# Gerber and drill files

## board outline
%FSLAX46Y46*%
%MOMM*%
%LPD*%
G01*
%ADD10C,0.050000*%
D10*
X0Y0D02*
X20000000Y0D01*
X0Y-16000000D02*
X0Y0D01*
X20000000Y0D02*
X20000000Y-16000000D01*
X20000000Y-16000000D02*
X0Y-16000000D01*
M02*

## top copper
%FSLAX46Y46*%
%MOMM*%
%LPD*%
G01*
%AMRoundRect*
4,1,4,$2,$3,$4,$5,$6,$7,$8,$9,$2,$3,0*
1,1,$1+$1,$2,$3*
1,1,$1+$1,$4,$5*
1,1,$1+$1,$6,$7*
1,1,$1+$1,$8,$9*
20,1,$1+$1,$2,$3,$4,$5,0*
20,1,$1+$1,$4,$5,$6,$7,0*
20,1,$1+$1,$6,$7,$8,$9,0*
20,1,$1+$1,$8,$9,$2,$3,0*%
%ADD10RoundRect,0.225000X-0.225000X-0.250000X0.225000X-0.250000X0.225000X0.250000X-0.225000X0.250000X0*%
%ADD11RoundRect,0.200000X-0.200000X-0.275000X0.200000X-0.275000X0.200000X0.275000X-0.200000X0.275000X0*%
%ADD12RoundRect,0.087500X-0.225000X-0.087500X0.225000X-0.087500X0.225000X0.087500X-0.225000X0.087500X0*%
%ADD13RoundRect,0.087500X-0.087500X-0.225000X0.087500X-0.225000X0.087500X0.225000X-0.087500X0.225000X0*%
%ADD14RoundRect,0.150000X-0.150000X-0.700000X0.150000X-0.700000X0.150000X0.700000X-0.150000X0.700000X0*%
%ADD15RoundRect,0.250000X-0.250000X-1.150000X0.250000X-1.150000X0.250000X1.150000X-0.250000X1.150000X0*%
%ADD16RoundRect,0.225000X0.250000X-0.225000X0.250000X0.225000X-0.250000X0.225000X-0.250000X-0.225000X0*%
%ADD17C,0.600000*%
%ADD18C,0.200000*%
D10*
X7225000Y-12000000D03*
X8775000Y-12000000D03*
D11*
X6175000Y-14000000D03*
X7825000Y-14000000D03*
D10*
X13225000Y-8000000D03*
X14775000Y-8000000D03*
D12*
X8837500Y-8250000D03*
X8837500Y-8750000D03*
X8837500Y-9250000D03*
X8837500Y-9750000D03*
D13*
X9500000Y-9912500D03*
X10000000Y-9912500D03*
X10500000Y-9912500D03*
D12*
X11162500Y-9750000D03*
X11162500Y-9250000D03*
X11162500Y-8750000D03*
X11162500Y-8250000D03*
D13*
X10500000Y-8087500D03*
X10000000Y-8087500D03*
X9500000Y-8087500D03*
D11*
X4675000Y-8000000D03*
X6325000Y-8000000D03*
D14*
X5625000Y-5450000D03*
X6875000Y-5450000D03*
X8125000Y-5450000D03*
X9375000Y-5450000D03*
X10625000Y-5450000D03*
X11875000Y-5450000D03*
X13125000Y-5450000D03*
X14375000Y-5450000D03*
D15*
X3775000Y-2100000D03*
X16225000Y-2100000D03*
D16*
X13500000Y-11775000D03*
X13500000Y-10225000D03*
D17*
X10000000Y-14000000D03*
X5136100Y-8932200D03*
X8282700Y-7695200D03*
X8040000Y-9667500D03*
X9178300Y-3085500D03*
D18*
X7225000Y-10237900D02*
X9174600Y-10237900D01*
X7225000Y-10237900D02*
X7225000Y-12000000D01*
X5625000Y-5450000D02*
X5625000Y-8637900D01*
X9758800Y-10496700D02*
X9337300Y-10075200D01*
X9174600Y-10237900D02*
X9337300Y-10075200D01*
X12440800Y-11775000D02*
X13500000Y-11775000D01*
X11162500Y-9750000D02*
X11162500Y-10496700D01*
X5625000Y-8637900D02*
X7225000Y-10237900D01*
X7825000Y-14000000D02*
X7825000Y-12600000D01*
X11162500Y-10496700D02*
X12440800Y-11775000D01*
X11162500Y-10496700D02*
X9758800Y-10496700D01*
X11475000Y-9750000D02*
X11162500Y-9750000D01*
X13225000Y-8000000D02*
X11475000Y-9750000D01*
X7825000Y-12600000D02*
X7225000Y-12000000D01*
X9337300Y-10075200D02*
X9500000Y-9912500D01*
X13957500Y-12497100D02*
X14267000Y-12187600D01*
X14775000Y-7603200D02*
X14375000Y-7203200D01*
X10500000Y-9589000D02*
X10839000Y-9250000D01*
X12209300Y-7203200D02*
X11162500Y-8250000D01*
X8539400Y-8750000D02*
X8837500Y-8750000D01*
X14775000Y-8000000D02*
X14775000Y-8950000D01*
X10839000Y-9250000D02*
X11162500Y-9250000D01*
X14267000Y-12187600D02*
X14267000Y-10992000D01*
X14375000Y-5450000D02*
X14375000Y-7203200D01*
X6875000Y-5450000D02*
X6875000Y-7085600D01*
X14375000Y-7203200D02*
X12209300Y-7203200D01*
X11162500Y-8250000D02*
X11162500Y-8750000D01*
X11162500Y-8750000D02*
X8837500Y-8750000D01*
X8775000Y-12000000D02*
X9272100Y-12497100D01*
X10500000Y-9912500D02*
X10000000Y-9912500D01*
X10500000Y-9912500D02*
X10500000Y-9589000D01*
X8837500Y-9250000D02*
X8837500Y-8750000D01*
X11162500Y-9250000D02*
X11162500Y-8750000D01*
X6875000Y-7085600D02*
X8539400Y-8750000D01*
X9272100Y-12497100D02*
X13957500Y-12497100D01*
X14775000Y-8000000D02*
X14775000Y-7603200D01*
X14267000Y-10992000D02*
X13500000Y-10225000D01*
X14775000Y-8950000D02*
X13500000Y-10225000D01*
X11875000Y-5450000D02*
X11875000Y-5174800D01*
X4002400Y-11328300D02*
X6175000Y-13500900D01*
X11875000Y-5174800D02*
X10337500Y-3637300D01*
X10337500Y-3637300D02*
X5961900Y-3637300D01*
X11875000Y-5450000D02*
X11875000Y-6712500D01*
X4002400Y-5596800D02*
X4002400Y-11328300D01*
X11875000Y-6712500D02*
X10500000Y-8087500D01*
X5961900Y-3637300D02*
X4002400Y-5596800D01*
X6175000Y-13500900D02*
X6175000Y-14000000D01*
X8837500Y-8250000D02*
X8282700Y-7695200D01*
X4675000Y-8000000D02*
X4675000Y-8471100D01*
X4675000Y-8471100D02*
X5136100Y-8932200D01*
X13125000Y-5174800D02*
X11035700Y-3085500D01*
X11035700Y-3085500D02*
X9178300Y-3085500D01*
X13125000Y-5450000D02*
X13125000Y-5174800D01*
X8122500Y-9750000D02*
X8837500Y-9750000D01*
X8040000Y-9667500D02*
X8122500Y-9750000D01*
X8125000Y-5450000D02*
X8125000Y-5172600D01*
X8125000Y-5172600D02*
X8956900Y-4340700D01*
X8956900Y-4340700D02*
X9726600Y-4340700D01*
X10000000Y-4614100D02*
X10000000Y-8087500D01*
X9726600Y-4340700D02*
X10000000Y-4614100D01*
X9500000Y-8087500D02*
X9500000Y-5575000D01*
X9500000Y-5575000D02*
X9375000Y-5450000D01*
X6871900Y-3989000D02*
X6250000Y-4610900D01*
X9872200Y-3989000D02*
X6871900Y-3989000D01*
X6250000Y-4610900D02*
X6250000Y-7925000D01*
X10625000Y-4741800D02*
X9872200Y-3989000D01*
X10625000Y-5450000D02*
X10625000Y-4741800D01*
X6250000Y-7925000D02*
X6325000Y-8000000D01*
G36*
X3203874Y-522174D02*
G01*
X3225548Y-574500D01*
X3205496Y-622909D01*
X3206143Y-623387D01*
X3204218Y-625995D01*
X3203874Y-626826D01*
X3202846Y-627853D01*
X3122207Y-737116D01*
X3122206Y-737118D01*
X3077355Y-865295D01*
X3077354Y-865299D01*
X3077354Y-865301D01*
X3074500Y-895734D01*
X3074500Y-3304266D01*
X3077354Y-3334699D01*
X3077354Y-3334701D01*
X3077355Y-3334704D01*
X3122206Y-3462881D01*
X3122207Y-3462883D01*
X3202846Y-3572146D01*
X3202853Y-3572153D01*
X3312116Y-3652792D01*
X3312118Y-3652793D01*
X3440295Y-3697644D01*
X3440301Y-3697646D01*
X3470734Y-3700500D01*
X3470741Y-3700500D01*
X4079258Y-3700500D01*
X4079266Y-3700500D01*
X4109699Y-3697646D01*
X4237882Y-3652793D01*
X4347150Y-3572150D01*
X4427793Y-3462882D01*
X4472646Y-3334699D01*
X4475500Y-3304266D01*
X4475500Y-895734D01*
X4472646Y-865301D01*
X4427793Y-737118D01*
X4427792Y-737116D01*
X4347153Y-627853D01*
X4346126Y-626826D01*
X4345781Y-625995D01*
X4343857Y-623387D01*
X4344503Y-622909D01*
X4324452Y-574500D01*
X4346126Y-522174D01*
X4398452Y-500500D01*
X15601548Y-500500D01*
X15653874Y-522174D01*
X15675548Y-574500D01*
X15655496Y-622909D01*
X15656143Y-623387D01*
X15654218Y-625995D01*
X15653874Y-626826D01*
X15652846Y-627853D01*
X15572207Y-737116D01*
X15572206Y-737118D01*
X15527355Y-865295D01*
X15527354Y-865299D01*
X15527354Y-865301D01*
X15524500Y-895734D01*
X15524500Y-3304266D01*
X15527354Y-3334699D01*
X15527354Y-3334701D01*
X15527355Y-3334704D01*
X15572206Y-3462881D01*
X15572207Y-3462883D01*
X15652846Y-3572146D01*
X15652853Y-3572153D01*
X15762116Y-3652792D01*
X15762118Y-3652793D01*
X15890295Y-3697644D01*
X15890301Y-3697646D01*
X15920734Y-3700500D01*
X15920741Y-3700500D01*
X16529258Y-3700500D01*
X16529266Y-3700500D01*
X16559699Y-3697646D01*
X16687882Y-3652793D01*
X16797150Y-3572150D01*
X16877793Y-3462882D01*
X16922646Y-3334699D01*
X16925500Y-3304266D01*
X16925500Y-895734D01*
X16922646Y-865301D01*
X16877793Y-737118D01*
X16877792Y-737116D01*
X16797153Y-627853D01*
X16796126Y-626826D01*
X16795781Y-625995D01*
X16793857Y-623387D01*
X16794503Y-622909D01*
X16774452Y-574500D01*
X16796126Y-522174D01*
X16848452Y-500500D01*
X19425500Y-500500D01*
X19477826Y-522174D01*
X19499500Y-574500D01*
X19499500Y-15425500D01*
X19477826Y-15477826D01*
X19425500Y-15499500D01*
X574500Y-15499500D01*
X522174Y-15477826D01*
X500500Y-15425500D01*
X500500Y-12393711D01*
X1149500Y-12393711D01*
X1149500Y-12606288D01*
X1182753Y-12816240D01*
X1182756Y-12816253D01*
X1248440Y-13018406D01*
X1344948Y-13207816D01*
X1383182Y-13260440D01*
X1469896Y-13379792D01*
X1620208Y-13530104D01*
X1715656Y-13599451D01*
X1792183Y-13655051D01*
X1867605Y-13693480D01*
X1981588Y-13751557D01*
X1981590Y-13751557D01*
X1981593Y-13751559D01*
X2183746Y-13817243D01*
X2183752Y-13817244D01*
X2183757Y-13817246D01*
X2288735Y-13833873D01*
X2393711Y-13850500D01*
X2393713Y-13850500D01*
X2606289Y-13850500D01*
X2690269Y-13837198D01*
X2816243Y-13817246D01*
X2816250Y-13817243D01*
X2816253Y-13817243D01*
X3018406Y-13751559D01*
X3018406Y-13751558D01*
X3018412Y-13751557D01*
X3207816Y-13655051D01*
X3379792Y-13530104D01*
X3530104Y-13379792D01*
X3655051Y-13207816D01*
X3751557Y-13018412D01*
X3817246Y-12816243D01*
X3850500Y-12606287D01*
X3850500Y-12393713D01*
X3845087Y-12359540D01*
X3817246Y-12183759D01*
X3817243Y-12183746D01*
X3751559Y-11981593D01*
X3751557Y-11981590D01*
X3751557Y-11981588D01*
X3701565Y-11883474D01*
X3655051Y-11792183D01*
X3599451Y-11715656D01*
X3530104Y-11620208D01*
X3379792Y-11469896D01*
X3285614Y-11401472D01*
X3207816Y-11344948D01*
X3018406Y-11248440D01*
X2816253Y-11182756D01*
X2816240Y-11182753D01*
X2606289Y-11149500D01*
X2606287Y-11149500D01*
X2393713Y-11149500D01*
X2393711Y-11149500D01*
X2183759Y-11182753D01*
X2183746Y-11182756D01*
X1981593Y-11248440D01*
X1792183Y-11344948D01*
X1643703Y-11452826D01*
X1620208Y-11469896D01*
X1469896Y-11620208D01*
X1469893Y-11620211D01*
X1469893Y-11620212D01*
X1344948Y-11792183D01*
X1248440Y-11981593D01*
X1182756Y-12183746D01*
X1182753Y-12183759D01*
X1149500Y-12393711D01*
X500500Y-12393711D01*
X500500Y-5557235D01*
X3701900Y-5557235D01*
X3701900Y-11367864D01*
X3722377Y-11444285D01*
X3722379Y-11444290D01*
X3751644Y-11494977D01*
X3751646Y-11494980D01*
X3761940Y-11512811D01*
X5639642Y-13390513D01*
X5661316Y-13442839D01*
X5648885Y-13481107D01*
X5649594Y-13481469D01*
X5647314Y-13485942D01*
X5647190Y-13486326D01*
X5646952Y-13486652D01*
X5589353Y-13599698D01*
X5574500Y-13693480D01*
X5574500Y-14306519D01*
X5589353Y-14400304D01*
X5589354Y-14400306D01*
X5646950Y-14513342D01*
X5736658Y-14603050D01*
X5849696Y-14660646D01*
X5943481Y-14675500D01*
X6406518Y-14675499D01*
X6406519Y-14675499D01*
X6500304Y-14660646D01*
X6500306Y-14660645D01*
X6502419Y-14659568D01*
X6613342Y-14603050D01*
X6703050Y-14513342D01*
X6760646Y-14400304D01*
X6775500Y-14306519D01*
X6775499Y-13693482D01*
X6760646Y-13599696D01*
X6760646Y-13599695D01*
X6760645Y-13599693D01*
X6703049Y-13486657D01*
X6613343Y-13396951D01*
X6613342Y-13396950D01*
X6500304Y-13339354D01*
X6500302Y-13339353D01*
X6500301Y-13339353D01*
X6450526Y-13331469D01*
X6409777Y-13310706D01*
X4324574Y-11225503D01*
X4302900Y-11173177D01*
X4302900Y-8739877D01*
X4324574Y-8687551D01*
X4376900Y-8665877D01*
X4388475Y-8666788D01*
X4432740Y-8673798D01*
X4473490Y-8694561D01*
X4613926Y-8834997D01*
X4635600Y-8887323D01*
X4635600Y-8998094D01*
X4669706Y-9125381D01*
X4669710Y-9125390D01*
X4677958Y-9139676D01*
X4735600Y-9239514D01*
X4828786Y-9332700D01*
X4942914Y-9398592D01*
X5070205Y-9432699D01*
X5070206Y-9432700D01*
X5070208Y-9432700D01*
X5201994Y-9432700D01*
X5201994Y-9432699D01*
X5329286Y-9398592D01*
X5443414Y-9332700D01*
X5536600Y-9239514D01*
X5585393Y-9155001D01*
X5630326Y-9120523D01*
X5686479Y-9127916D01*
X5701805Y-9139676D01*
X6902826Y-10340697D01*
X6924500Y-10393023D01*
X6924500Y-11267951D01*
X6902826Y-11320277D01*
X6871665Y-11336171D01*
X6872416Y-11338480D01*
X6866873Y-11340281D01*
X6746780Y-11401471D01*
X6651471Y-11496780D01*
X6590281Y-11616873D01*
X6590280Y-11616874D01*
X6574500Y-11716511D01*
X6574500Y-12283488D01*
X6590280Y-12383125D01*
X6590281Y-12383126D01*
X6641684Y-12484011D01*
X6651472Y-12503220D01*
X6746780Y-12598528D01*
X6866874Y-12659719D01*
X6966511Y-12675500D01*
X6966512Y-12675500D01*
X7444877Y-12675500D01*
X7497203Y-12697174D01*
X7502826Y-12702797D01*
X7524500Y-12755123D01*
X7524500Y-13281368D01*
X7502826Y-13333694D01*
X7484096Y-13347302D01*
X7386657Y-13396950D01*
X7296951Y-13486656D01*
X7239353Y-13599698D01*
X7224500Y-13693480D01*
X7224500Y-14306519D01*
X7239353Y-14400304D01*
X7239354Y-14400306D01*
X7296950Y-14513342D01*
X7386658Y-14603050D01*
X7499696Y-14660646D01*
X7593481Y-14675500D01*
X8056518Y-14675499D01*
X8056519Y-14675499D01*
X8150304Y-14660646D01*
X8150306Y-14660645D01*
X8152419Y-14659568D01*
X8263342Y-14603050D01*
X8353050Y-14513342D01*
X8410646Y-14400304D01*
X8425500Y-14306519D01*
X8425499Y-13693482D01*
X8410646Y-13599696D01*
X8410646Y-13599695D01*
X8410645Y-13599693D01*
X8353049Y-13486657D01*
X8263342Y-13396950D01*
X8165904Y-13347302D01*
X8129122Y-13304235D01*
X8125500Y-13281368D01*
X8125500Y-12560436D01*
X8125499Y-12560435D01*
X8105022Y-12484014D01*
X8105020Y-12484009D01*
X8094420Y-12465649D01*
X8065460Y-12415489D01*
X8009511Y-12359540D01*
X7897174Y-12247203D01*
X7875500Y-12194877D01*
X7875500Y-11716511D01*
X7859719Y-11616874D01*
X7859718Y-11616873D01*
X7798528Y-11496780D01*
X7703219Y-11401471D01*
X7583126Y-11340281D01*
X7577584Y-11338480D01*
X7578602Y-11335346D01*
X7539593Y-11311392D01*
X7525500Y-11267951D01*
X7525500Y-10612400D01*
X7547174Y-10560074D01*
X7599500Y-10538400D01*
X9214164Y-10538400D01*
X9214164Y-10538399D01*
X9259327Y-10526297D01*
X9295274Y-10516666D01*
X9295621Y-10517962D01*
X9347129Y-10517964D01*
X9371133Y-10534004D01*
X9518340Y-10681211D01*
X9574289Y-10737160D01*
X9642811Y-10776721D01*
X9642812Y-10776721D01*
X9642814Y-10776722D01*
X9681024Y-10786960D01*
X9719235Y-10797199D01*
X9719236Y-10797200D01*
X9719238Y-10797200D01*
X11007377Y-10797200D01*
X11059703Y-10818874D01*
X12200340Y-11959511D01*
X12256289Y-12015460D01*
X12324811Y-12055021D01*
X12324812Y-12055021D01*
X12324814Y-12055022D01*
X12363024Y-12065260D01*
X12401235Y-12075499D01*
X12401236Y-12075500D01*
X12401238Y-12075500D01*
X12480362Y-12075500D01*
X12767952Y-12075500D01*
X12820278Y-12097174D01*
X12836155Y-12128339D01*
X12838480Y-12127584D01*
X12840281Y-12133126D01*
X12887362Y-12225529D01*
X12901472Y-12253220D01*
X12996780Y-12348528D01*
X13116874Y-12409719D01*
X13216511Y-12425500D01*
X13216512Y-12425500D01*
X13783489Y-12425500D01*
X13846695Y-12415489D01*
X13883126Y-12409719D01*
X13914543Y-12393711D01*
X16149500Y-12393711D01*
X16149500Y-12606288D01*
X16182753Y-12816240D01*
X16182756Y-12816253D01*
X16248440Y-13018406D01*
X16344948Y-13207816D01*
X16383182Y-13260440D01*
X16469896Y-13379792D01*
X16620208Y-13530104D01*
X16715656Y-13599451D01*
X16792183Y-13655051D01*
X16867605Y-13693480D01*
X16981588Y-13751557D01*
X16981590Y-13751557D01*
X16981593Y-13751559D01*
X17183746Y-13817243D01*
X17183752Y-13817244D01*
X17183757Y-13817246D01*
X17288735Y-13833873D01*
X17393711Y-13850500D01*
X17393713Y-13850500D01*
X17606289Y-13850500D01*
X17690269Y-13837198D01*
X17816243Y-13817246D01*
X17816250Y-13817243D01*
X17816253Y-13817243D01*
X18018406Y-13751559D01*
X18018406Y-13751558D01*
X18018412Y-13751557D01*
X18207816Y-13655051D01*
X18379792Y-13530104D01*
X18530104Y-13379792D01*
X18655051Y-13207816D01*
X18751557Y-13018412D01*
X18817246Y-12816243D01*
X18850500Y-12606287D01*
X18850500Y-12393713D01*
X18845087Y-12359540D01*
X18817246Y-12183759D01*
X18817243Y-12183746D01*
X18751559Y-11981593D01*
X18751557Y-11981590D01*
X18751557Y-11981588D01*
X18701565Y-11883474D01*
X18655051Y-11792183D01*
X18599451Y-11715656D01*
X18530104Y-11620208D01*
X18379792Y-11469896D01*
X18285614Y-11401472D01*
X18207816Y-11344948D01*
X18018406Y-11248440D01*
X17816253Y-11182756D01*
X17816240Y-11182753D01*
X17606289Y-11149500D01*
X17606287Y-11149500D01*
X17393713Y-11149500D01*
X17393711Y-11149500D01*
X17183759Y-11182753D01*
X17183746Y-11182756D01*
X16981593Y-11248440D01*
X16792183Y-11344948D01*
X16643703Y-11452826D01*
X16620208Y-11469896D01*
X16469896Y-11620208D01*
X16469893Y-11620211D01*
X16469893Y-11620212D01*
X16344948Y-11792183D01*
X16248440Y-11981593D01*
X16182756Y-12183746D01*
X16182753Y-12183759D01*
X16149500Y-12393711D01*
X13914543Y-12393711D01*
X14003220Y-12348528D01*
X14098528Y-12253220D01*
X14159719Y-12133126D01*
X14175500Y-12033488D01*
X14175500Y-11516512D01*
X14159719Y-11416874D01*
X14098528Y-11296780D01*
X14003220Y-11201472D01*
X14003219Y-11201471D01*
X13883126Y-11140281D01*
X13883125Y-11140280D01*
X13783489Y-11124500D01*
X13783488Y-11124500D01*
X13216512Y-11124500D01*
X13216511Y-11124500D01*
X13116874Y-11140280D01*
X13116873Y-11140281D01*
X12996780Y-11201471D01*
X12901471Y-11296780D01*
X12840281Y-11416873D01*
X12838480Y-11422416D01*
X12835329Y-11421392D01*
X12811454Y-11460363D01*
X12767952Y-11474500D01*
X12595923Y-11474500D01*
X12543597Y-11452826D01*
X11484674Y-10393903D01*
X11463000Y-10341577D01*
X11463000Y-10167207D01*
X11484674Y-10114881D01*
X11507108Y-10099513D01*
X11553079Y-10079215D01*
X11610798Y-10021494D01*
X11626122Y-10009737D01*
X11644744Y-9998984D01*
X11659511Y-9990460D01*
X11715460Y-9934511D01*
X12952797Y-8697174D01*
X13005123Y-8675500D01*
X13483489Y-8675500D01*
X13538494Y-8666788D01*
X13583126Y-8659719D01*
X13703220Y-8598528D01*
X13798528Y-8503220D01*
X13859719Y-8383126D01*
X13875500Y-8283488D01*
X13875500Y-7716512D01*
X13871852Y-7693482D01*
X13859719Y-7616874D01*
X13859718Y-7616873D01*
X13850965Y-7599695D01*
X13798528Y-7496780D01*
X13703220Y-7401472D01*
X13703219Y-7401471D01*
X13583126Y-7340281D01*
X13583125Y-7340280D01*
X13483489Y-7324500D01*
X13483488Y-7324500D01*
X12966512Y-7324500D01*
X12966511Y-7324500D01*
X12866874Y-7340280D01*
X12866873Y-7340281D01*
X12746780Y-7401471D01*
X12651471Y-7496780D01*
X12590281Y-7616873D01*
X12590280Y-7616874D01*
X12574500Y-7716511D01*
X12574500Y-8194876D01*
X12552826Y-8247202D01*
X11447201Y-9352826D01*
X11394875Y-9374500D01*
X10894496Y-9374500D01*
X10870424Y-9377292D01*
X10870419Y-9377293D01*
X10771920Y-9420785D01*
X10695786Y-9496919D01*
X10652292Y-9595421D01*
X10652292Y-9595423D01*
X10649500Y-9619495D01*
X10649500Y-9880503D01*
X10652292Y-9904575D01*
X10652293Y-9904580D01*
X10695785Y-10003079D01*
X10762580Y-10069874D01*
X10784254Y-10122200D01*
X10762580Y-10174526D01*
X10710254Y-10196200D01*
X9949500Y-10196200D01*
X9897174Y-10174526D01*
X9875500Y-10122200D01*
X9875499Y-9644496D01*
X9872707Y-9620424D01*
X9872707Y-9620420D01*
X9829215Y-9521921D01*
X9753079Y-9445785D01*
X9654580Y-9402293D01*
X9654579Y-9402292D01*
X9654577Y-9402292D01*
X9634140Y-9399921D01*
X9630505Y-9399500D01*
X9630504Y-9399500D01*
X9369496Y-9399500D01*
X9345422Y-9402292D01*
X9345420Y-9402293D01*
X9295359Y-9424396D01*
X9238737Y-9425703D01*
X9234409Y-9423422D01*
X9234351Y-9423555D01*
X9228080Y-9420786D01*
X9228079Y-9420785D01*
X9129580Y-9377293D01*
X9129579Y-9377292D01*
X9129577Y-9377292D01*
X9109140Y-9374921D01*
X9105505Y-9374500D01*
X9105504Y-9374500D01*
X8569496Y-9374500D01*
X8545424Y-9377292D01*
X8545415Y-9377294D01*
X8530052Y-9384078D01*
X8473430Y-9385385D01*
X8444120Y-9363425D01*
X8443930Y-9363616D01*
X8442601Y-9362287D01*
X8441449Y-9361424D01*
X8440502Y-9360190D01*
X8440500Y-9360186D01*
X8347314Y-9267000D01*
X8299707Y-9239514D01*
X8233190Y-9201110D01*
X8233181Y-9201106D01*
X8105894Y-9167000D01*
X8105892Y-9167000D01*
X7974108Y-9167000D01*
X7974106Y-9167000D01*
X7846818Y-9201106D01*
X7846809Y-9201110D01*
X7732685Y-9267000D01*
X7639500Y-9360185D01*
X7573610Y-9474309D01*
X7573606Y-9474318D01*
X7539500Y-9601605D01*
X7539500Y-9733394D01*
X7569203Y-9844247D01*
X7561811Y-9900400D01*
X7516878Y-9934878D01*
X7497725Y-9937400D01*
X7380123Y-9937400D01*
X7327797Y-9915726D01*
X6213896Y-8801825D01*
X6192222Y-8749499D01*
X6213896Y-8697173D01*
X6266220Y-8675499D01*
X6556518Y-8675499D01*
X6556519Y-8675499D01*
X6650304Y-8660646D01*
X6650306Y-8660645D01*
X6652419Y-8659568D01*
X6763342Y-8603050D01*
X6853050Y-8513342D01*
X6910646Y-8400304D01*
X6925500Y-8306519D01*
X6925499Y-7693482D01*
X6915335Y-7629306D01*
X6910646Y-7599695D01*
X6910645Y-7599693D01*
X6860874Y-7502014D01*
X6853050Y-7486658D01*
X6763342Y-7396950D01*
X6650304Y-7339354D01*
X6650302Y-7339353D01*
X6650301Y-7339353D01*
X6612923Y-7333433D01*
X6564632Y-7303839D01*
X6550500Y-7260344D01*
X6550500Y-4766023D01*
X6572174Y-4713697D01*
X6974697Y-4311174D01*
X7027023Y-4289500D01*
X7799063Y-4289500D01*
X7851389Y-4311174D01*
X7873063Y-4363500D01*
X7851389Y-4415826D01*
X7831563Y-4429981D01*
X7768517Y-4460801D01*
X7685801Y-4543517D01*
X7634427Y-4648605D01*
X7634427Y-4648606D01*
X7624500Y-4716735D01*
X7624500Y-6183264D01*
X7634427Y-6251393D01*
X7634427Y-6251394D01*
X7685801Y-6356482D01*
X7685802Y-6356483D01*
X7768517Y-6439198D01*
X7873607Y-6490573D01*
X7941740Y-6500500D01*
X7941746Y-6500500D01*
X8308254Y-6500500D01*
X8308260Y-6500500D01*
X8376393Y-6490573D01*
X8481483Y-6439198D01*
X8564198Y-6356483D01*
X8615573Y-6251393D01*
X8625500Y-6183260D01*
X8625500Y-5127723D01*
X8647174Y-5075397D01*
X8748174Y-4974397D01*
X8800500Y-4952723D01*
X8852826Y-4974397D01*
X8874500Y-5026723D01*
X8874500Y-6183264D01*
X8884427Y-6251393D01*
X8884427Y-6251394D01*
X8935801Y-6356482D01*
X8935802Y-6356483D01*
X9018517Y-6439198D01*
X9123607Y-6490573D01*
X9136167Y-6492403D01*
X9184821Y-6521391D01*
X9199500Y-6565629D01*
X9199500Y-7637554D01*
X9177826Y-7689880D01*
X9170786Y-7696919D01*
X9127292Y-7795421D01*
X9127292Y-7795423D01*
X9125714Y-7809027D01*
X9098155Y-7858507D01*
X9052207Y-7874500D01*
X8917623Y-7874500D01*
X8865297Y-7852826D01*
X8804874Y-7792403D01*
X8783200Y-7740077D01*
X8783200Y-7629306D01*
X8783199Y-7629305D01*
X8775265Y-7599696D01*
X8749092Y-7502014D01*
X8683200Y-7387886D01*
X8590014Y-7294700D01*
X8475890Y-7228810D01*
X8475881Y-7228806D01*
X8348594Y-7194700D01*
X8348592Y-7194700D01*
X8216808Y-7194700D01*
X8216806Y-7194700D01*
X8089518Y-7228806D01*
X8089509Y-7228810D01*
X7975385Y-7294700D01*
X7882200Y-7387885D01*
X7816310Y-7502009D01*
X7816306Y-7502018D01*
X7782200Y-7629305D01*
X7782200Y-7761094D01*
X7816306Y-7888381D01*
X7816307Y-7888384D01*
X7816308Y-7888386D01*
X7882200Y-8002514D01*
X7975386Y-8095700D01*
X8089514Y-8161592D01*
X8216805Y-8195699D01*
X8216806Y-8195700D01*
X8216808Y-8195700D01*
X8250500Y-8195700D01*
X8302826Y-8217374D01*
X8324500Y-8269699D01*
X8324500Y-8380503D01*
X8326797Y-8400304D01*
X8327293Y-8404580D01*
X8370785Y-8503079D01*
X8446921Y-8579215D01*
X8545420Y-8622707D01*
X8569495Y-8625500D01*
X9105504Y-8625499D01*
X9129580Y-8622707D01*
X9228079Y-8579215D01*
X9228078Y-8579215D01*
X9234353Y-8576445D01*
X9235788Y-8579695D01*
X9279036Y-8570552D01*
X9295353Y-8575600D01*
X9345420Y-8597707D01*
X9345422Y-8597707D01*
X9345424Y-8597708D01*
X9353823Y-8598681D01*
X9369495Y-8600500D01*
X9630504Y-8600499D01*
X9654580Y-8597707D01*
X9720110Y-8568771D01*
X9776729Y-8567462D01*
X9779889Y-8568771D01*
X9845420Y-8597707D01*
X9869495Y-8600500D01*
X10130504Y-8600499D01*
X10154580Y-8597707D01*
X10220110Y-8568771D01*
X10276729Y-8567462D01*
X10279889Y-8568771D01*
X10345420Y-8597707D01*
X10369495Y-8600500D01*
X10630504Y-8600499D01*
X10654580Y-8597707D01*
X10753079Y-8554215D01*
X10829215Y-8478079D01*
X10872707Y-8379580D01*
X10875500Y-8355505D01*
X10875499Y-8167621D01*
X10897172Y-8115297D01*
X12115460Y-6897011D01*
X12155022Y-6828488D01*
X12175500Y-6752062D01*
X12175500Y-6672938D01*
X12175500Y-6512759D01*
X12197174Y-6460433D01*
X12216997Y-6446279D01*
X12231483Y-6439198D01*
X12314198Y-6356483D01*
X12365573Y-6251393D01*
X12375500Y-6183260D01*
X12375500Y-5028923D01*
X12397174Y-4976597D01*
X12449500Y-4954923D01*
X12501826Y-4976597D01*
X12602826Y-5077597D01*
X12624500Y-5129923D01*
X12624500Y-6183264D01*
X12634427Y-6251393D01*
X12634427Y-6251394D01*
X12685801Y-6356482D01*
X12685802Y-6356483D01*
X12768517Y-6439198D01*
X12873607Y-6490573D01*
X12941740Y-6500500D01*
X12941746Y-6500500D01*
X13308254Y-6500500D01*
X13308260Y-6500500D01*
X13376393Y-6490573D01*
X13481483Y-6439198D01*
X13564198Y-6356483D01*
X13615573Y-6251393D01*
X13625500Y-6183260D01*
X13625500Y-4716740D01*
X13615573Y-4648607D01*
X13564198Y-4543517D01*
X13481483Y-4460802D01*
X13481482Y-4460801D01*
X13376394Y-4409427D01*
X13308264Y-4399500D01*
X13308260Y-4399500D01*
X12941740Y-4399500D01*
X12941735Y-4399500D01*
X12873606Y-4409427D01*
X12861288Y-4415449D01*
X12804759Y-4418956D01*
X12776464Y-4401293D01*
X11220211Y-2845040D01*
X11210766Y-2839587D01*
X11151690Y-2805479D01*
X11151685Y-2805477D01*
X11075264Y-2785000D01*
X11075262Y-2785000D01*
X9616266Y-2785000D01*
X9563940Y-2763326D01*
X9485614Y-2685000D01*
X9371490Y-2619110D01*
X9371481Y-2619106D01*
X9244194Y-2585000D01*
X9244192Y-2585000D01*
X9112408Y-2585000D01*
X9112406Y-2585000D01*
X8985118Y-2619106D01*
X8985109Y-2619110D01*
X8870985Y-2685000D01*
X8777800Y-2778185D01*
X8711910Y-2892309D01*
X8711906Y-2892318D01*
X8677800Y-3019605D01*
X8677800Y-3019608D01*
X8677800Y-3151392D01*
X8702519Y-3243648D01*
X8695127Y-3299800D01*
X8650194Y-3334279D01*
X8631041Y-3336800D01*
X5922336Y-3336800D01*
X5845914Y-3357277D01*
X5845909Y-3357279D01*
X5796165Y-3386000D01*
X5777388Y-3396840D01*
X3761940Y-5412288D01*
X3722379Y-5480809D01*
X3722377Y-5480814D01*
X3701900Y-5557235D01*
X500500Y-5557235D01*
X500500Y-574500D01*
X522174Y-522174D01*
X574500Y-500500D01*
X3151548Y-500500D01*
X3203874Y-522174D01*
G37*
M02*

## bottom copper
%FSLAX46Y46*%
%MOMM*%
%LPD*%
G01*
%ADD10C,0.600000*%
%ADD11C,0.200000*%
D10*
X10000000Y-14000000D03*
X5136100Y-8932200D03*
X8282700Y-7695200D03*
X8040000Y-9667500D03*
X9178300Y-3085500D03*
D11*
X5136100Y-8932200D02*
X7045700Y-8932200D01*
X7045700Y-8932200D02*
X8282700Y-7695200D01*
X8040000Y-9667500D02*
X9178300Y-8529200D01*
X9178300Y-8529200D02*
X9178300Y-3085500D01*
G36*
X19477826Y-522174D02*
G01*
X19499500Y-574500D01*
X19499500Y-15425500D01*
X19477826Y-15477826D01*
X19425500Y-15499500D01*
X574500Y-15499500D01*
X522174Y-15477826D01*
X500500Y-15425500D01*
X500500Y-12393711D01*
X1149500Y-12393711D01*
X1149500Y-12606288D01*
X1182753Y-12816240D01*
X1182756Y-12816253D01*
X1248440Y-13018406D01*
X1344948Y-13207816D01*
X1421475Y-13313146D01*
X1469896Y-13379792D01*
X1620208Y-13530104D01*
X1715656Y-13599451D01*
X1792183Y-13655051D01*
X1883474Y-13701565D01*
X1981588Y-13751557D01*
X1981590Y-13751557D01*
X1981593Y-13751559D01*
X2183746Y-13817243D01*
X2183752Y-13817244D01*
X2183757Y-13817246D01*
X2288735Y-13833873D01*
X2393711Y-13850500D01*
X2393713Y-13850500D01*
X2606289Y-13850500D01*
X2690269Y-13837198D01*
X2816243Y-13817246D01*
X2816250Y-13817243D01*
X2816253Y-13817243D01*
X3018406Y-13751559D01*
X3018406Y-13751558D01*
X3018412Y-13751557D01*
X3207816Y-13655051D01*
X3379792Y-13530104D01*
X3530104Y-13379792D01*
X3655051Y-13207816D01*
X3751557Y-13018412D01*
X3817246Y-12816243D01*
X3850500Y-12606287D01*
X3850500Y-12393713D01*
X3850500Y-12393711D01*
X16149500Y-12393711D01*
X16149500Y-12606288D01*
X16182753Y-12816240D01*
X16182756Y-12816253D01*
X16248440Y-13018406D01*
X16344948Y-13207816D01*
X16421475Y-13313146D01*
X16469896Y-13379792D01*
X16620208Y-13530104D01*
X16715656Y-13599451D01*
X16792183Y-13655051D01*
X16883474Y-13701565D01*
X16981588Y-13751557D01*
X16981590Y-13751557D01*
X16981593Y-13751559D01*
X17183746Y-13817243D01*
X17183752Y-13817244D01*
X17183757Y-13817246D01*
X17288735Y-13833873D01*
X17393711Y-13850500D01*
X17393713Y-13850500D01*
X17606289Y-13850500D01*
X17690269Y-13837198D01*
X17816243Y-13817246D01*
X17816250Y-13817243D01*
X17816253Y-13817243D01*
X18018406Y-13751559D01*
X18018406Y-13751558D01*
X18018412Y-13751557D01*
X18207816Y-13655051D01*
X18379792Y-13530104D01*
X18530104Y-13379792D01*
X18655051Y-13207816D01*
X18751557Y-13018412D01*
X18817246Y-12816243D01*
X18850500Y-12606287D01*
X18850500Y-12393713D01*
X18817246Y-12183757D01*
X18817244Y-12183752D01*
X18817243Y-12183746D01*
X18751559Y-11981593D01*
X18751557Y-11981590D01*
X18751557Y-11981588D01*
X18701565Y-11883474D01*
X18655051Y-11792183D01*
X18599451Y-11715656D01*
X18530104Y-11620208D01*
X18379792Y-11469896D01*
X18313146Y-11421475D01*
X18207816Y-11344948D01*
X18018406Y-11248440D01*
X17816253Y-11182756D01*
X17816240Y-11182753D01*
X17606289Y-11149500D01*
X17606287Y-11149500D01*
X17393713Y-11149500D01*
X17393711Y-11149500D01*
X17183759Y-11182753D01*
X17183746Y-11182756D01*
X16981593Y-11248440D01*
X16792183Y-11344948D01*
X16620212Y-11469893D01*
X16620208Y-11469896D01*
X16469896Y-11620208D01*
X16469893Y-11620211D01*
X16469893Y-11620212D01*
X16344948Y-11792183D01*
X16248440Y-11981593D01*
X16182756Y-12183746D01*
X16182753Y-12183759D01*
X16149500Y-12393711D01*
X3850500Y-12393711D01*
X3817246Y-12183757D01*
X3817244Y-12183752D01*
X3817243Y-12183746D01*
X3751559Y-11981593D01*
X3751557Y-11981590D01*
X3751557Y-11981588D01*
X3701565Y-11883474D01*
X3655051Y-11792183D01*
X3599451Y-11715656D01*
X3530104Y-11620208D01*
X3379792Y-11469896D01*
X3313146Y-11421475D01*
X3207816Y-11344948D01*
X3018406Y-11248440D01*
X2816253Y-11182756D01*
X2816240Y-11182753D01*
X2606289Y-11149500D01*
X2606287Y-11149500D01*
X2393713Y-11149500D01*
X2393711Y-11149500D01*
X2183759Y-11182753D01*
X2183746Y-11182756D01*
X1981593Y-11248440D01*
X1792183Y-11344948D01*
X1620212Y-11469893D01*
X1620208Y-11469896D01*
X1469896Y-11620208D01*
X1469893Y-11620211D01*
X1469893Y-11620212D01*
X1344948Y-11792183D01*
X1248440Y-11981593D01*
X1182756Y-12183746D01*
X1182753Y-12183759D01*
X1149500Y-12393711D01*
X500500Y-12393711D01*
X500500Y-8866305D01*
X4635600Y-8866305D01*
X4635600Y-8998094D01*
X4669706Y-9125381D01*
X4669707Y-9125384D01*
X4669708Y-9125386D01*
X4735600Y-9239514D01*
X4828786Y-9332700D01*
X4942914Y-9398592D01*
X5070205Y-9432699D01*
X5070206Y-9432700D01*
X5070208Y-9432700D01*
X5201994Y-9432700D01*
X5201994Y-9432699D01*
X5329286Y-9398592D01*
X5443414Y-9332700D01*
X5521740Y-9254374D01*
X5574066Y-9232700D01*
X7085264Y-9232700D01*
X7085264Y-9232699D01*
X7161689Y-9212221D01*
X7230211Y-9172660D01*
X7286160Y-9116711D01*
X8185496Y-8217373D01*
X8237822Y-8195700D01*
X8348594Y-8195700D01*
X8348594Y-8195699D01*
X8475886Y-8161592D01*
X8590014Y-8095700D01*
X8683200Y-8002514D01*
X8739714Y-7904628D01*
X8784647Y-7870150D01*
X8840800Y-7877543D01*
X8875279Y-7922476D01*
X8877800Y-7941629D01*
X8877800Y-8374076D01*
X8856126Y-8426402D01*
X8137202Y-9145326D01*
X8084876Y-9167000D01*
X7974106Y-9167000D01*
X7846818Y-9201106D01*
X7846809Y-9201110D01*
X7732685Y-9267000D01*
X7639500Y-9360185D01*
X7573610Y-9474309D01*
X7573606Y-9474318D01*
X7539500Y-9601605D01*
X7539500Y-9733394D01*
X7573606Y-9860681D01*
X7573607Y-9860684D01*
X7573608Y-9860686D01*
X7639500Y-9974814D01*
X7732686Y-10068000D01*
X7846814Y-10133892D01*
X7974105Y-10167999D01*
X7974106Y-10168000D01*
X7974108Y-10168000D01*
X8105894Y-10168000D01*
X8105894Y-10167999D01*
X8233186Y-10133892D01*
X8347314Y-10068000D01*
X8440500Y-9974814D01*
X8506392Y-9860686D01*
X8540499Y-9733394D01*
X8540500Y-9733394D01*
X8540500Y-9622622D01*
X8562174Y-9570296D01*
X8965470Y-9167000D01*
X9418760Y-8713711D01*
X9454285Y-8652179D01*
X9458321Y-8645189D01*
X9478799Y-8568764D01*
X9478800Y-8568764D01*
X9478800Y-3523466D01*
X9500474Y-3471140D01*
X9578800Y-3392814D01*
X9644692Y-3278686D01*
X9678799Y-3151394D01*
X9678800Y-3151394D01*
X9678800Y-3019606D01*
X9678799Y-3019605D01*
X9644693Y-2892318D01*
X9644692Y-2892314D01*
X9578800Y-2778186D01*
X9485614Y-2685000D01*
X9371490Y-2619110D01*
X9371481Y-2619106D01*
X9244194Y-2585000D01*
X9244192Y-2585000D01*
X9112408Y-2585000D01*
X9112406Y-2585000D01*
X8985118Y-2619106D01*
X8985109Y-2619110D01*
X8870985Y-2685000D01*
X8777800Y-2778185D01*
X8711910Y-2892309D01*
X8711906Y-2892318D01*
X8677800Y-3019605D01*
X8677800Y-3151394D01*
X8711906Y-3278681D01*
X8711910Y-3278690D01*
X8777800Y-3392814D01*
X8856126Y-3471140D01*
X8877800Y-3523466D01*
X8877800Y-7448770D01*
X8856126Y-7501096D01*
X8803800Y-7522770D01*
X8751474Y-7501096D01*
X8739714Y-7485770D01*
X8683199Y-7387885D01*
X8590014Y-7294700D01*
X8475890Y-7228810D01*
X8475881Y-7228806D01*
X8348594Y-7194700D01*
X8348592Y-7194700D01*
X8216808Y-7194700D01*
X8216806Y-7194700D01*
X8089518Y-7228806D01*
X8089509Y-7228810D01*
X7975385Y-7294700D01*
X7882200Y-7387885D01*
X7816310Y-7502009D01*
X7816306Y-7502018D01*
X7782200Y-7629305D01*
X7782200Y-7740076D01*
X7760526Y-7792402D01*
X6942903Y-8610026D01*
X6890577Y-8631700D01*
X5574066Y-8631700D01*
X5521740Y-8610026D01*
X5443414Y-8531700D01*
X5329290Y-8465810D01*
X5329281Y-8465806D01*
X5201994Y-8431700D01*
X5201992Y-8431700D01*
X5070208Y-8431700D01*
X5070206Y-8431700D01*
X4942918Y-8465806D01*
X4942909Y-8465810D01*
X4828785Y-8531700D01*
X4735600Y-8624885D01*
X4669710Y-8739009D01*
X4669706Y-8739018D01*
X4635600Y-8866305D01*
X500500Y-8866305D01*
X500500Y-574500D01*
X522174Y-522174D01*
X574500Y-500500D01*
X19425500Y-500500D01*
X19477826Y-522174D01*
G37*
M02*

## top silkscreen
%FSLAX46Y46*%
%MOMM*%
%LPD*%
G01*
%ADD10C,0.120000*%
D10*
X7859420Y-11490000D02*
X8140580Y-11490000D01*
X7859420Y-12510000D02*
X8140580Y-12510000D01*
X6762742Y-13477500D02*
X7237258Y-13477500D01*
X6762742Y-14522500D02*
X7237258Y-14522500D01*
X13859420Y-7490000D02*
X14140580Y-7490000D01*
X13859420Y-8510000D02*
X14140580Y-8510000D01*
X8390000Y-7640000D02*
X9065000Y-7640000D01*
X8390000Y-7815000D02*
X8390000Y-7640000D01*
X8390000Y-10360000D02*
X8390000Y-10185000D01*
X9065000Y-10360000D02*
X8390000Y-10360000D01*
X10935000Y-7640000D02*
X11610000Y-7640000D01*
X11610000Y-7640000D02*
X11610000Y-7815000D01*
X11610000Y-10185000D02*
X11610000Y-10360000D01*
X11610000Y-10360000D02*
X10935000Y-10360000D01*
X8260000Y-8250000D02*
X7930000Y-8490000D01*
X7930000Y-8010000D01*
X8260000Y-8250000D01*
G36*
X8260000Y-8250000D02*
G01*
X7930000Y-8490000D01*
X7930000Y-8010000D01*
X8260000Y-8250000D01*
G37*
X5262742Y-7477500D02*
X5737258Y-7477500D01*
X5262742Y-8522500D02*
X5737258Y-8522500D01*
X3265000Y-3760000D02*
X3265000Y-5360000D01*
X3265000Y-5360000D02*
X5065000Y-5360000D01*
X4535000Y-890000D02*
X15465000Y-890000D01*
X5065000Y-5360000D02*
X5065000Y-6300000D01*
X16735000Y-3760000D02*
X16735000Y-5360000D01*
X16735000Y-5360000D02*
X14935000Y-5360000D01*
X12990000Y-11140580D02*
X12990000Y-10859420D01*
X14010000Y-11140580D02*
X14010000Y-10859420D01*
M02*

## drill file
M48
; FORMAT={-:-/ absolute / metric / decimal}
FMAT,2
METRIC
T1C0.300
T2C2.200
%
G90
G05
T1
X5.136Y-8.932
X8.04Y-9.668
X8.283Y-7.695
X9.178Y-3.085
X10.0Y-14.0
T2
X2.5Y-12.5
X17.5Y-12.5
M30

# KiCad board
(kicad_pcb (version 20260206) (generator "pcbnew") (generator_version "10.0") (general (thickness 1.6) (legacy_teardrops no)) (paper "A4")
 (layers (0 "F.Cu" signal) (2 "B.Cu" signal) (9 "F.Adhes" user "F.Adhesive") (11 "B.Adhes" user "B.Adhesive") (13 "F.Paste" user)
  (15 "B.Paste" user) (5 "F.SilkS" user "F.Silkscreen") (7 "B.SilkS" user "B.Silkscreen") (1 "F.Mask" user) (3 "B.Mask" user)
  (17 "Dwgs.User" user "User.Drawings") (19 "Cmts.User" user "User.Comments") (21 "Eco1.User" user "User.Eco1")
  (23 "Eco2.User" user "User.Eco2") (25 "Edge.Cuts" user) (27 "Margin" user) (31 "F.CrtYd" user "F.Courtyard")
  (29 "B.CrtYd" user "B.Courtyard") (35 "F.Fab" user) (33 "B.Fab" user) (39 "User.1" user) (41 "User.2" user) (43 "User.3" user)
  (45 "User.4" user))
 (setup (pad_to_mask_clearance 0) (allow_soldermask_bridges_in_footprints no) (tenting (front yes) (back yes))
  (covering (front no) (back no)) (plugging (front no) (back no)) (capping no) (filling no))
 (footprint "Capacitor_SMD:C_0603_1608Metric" (layer "F.Cu") (at 8 12)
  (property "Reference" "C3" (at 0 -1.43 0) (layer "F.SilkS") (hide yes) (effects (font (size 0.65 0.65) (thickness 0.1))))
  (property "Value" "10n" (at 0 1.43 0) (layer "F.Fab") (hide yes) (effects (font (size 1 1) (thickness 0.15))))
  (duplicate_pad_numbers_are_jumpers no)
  (fp_line (start -0.14058 -0.51) (end 0.14058 -0.51) (stroke (width 0.12) (type solid)) (layer "F.SilkS"))
  (fp_line (start -0.14058 0.51) (end 0.14058 0.51) (stroke (width 0.12) (type solid)) (layer "F.SilkS"))
  (pad "1" smd roundrect (at -0.775 0) (size 0.9 0.95) (layers "F.Cu" "F.Mask" "F.Paste") (roundrect_rratio 0.25) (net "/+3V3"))
  (pad "2" smd roundrect (at 0.775 0) (size 0.9 0.95) (layers "F.Cu" "F.Mask" "F.Paste") (roundrect_rratio 0.25) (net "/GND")
   (zone_connect 2)))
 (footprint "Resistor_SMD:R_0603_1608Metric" (layer "F.Cu") (at 7 14)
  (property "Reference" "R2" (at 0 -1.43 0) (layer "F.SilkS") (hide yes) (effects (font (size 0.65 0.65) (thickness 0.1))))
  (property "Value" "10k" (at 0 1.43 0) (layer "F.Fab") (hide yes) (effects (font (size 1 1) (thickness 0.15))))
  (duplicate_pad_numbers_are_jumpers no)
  (fp_line (start -0.237258 -0.5225) (end 0.237258 -0.5225) (stroke (width 0.12) (type solid)) (layer "F.SilkS"))
  (fp_line (start -0.237258 0.5225) (end 0.237258 0.5225) (stroke (width 0.12) (type solid)) (layer "F.SilkS"))
  (pad "1" smd roundrect (at -0.825 0) (size 0.8 0.95) (layers "F.Cu" "F.Mask" "F.Paste") (roundrect_rratio 0.25) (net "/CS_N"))
  (pad "2" smd roundrect (at 0.825 0) (size 0.8 0.95) (layers "F.Cu" "F.Mask" "F.Paste") (roundrect_rratio 0.25) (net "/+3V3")))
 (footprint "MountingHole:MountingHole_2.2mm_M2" (layer "F.Cu") (at 2.5 12.5)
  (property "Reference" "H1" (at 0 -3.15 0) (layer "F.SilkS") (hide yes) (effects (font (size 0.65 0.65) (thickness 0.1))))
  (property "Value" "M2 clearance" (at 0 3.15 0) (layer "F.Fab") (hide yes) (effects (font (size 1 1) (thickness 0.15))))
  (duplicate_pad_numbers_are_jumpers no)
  (pad "" np_thru_hole circle (at 0 0) (size 2.2 2.2) (drill 2.2) (layers "*.Cu" "*.Mask")))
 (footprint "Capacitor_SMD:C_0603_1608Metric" (layer "F.Cu") (at 14 8)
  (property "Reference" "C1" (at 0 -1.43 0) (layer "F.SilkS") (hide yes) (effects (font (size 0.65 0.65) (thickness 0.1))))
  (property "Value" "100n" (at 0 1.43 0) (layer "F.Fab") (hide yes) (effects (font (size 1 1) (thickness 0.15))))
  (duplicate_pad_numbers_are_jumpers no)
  (fp_line (start -0.14058 -0.51) (end 0.14058 -0.51) (stroke (width 0.12) (type solid)) (layer "F.SilkS"))
  (fp_line (start -0.14058 0.51) (end 0.14058 0.51) (stroke (width 0.12) (type solid)) (layer "F.SilkS"))
  (pad "1" smd roundrect (at -0.775 0) (size 0.9 0.95) (layers "F.Cu" "F.Mask" "F.Paste") (roundrect_rratio 0.25) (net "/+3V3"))
  (pad "2" smd roundrect (at 0.775 0) (size 0.9 0.95) (layers "F.Cu" "F.Mask" "F.Paste") (roundrect_rratio 0.25) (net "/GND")
   (zone_connect 2)))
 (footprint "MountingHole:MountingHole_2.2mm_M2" (layer "F.Cu") (at 17.5 12.5)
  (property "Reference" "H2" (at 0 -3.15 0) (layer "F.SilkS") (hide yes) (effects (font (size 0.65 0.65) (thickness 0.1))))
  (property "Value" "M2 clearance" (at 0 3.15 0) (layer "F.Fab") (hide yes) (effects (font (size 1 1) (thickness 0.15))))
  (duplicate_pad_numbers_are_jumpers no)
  (pad "" np_thru_hole circle (at 0 0) (size 2.2 2.2) (drill 2.2) (layers "*.Cu" "*.Mask")))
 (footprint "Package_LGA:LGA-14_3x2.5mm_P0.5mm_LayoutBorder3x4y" (layer "F.Cu") (at 10 9)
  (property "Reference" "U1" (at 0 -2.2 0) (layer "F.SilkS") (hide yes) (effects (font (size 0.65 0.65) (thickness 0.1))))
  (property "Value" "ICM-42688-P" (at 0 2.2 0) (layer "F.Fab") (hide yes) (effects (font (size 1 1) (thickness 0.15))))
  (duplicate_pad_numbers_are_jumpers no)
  (fp_line (start -1.61 -1.36) (end -0.935 -1.36) (stroke (width 0.12) (type solid)) (layer "F.SilkS"))
  (fp_line (start -1.61 -1.185) (end -1.61 -1.36) (stroke (width 0.12) (type solid)) (layer "F.SilkS"))
  (fp_line (start -1.61 1.36) (end -1.61 1.185) (stroke (width 0.12) (type solid)) (layer "F.SilkS"))
  (fp_line (start -0.935 1.36) (end -1.61 1.36) (stroke (width 0.12) (type solid)) (layer "F.SilkS"))
  (fp_line (start 0.935 -1.36) (end 1.61 -1.36) (stroke (width 0.12) (type solid)) (layer "F.SilkS"))
  (fp_line (start 1.61 -1.36) (end 1.61 -1.185) (stroke (width 0.12) (type solid)) (layer "F.SilkS"))
  (fp_line (start 1.61 1.185) (end 1.61 1.36) (stroke (width 0.12) (type solid)) (layer "F.SilkS"))
  (fp_line (start 1.61 1.36) (end 0.935 1.36) (stroke (width 0.12) (type solid)) (layer "F.SilkS"))
  (fp_poly (pts (xy -1.74 -0.75) (xy -2.07 -0.51) (xy -2.07 -0.99)) (stroke (width 0.12) (type solid)) (fill yes) (layer "F.SilkS"))
  (pad "1" smd roundrect (at -1.1625 -0.75) (size 0.625 0.35) (layers "F.Cu" "F.Mask" "F.Paste") (roundrect_rratio 0.25) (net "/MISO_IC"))
  (pad "2" smd roundrect (at -1.1625 -0.25) (size 0.625 0.35) (layers "F.Cu" "F.Mask" "F.Paste") (roundrect_rratio 0.25) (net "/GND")
   (zone_connect 2))
  (pad "3" smd roundrect (at -1.1625 0.25) (size 0.625 0.35) (layers "F.Cu" "F.Mask" "F.Paste") (roundrect_rratio 0.25) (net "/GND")
   (zone_connect 2))
  (pad "4" smd roundrect (at -1.1625 0.75) (size 0.625 0.35) (layers "F.Cu" "F.Mask" "F.Paste") (roundrect_rratio 0.25) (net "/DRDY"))
  (pad "5" smd roundrect (at -0.5 0.9125) (size 0.35 0.625) (layers "F.Cu" "F.Mask" "F.Paste") (roundrect_rratio 0.25) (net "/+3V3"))
  (pad "6" smd roundrect (at 0 0.9125) (size 0.35 0.625) (layers "F.Cu" "F.Mask" "F.Paste") (roundrect_rratio 0.25) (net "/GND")
   (zone_connect 2))
  (pad "7" smd roundrect (at 0.5 0.9125) (size 0.35 0.625) (layers "F.Cu" "F.Mask" "F.Paste") (roundrect_rratio 0.25) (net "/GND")
   (zone_connect 2))
  (pad "8" smd roundrect (at 1.1625 0.75) (size 0.625 0.35) (layers "F.Cu" "F.Mask" "F.Paste") (roundrect_rratio 0.25) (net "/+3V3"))
  (pad "9" smd roundrect (at 1.1625 0.25) (size 0.625 0.35) (layers "F.Cu" "F.Mask" "F.Paste") (roundrect_rratio 0.25) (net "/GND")
   (zone_connect 2))
  (pad "10" smd roundrect (at 1.1625 -0.25) (size 0.625 0.35) (layers "F.Cu" "F.Mask" "F.Paste") (roundrect_rratio 0.25) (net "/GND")
   (zone_connect 2))
  (pad "11" smd roundrect (at 1.1625 -0.75) (size 0.625 0.35) (layers "F.Cu" "F.Mask" "F.Paste") (roundrect_rratio 0.25) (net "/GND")
   (zone_connect 2))
  (pad "12" smd roundrect (at 0.5 -0.9125) (size 0.35 0.625) (layers "F.Cu" "F.Mask" "F.Paste") (roundrect_rratio 0.25) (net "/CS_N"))
  (pad "13" smd roundrect (at 0 -0.9125) (size 0.35 0.625) (layers "F.Cu" "F.Mask" "F.Paste") (roundrect_rratio 0.25) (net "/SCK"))
  (pad "14" smd roundrect (at -0.5 -0.9125) (size 0.35 0.625) (layers "F.Cu" "F.Mask" "F.Paste") (roundrect_rratio 0.25) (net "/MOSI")))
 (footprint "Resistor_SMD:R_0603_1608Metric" (layer "F.Cu") (at 5.5 8)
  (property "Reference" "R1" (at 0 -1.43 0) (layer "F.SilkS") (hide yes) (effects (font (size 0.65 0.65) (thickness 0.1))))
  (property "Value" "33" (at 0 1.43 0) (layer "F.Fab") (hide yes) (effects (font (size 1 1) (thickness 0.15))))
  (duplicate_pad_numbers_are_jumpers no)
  (fp_line (start -0.237258 -0.5225) (end 0.237258 -0.5225) (stroke (width 0.12) (type solid)) (layer "F.SilkS"))
  (fp_line (start -0.237258 0.5225) (end 0.237258 0.5225) (stroke (width 0.12) (type solid)) (layer "F.SilkS"))
  (pad "1" smd roundrect (at -0.825 0) (size 0.8 0.95) (layers "F.Cu" "F.Mask" "F.Paste") (roundrect_rratio 0.25) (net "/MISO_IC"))
  (pad "2" smd roundrect (at 0.825 0) (size 0.8 0.95) (layers "F.Cu" "F.Mask" "F.Paste") (roundrect_rratio 0.25) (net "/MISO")))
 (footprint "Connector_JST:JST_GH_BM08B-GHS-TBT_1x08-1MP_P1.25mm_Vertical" (layer "F.Cu") (at 10 3.5)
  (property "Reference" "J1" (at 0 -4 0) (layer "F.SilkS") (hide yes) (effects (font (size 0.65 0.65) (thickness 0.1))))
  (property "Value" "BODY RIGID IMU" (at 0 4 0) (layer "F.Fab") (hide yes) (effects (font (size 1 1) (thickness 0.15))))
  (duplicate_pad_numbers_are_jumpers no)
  (fp_line (start -6.735 0.26) (end -6.735 1.86) (stroke (width 0.12) (type solid)) (layer "F.SilkS"))
  (fp_line (start -6.735 1.86) (end -4.935 1.86) (stroke (width 0.12) (type solid)) (layer "F.SilkS"))
  (fp_line (start -5.465 -2.61) (end 5.465 -2.61) (stroke (width 0.12) (type solid)) (layer "F.SilkS"))
  (fp_line (start -4.935 1.86) (end -4.935 2.8) (stroke (width 0.12) (type solid)) (layer "F.SilkS"))
  (fp_line (start 6.735 0.26) (end 6.735 1.86) (stroke (width 0.12) (type solid)) (layer "F.SilkS"))
  (fp_line (start 6.735 1.86) (end 4.935 1.86) (stroke (width 0.12) (type solid)) (layer "F.SilkS"))
  (pad "1" smd roundrect (at -4.375 1.95) (size 0.6 1.7) (layers "F.Cu" "F.Mask" "F.Paste") (roundrect_rratio 0.25) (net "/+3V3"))
  (pad "2" smd roundrect (at -3.125 1.95) (size 0.6 1.7) (layers "F.Cu" "F.Mask" "F.Paste") (roundrect_rratio 0.25) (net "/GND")
   (zone_connect 2))
  (pad "3" smd roundrect (at -1.875 1.95) (size 0.6 1.7) (layers "F.Cu" "F.Mask" "F.Paste") (roundrect_rratio 0.25) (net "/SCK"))
  (pad "4" smd roundrect (at -0.625 1.95) (size 0.6 1.7) (layers "F.Cu" "F.Mask" "F.Paste") (roundrect_rratio 0.25) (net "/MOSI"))
  (pad "5" smd roundrect (at 0.625 1.95) (size 0.6 1.7) (layers "F.Cu" "F.Mask" "F.Paste") (roundrect_rratio 0.25) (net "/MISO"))
  (pad "6" smd roundrect (at 1.875 1.95) (size 0.6 1.7) (layers "F.Cu" "F.Mask" "F.Paste") (roundrect_rratio 0.25) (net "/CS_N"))
  (pad "7" smd roundrect (at 3.125 1.95) (size 0.6 1.7) (layers "F.Cu" "F.Mask" "F.Paste") (roundrect_rratio 0.25) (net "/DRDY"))
  (pad "8" smd roundrect (at 4.375 1.95) (size 0.6 1.7) (layers "F.Cu" "F.Mask" "F.Paste") (roundrect_rratio 0.25) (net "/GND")
   (zone_connect 2))
  (pad "MP" smd roundrect (at -6.225 -1.4) (size 1 2.8) (layers "F.Cu" "F.Mask" "F.Paste") (roundrect_rratio 0.25))
  (pad "MP" smd roundrect (at 6.225 -1.4) (size 1 2.8) (layers "F.Cu" "F.Mask" "F.Paste") (roundrect_rratio 0.25)))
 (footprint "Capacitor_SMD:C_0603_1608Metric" (layer "F.Cu") (at 13.5 11 90)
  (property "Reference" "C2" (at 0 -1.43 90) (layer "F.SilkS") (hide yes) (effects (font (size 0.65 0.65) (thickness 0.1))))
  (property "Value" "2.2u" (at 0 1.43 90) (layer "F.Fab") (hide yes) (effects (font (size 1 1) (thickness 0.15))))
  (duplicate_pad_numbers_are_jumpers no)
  (fp_line (start -0.14058 -0.51) (end 0.14058 -0.51) (stroke (width 0.12) (type solid)) (layer "F.SilkS"))
  (fp_line (start -0.14058 0.51) (end 0.14058 0.51) (stroke (width 0.12) (type solid)) (layer "F.SilkS"))
  (pad "1" smd roundrect (at -0.775 0 90) (size 0.9 0.95) (layers "F.Cu" "F.Mask" "F.Paste") (roundrect_rratio 0.25) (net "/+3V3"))
  (pad "2" smd roundrect (at 0.775 0 90) (size 0.9 0.95) (layers "F.Cu" "F.Mask" "F.Paste") (roundrect_rratio 0.25) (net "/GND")
   (zone_connect 2)))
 (gr_line (start 0 0) (end 20 0) (stroke (width 0.05) (type default)) (layer "Edge.Cuts"))
 (gr_line (start 0 16) (end 0 0) (stroke (width 0.05) (type default)) (layer "Edge.Cuts"))
 (gr_line (start 20 0) (end 20 16) (stroke (width 0.05) (type default)) (layer "Edge.Cuts"))
 (gr_line (start 20 16) (end 0 16) (stroke (width 0.05) (type default)) (layer "Edge.Cuts"))
 (segment (start 7.225 10.2379) (end 9.1746 10.2379) (width 0.2) (layer "F.Cu") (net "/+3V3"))
 (segment (start 7.225 10.2379) (end 7.225 12) (width 0.2) (layer "F.Cu") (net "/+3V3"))
 (segment (start 5.625 5.45) (end 5.625 8.6379) (width 0.2) (layer "F.Cu") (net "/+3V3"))
 (segment (start 9.7588 10.4967) (end 9.3373 10.0752) (width 0.2) (layer "F.Cu") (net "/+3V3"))
 (segment (start 9.1746 10.2379) (end 9.3373 10.0752) (width 0.2) (layer "F.Cu") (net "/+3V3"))
 (segment (start 12.4408 11.775) (end 13.5 11.775) (width 0.2) (layer "F.Cu") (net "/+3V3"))
 (segment (start 11.1625 9.75) (end 11.1625 10.4967) (width 0.2) (layer "F.Cu") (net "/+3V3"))
 (segment (start 5.625 8.6379) (end 7.225 10.2379) (width 0.2) (layer "F.Cu") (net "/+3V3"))
 (segment (start 7.825 14) (end 7.825 12.6) (width 0.2) (layer "F.Cu") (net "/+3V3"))
 (segment (start 11.1625 10.4967) (end 12.4408 11.775) (width 0.2) (layer "F.Cu") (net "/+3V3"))
 (segment (start 11.1625 10.4967) (end 9.7588 10.4967) (width 0.2) (layer "F.Cu") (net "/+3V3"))
 (segment (start 11.475 9.75) (end 11.1625 9.75) (width 0.2) (layer "F.Cu") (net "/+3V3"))
 (segment (start 13.225 8) (end 11.475 9.75) (width 0.2) (layer "F.Cu") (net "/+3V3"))
 (segment (start 7.825 12.6) (end 7.225 12) (width 0.2) (layer "F.Cu") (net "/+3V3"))
 (segment (start 9.3373 10.0752) (end 9.5 9.9125) (width 0.2) (layer "F.Cu") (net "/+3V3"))
 (segment (start 13.9575 12.4971) (end 14.267 12.1876) (width 0.2) (layer "F.Cu") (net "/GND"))
 (segment (start 14.775 7.6032) (end 14.375 7.2032) (width 0.2) (layer "F.Cu") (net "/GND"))
 (segment (start 10.5 9.589) (end 10.839 9.25) (width 0.2) (layer "F.Cu") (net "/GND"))
 (segment (start 12.2093 7.2032) (end 11.1625 8.25) (width 0.2) (layer "F.Cu") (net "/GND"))
 (segment (start 8.5394 8.75) (end 8.8375 8.75) (width 0.2) (layer "F.Cu") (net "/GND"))
 (segment (start 14.775 8) (end 14.775 8.95) (width 0.2) (layer "F.Cu") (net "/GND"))
 (segment (start 10.839 9.25) (end 11.1625 9.25) (width 0.2) (layer "F.Cu") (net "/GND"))
 (segment (start 14.267 12.1876) (end 14.267 10.992) (width 0.2) (layer "F.Cu") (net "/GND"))
 (segment (start 14.375 5.45) (end 14.375 7.2032) (width 0.2) (layer "F.Cu") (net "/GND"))
 (segment (start 6.875 5.45) (end 6.875 7.0856) (width 0.2) (layer "F.Cu") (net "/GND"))
 (segment (start 14.375 7.2032) (end 12.2093 7.2032) (width 0.2) (layer "F.Cu") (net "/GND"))
 (segment (start 11.1625 8.25) (end 11.1625 8.75) (width 0.2) (layer "F.Cu") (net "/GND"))
 (segment (start 11.1625 8.75) (end 8.8375 8.75) (width 0.2) (layer "F.Cu") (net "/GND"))
 (segment (start 8.775 12) (end 9.2721 12.4971) (width 0.2) (layer "F.Cu") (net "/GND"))
 (segment (start 10.5 9.9125) (end 10 9.9125) (width 0.2) (layer "F.Cu") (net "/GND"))
 (segment (start 10.5 9.9125) (end 10.5 9.589) (width 0.2) (layer "F.Cu") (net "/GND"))
 (segment (start 8.8375 9.25) (end 8.8375 8.75) (width 0.2) (layer "F.Cu") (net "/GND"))
 (segment (start 11.1625 9.25) (end 11.1625 8.75) (width 0.2) (layer "F.Cu") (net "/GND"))
 (segment (start 6.875 7.0856) (end 8.5394 8.75) (width 0.2) (layer "F.Cu") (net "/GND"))
 (segment (start 9.2721 12.4971) (end 13.9575 12.4971) (width 0.2) (layer "F.Cu") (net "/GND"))
 (segment (start 14.775 8) (end 14.775 7.6032) (width 0.2) (layer "F.Cu") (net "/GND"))
 (segment (start 14.267 10.992) (end 13.5 10.225) (width 0.2) (layer "F.Cu") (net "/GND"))
 (segment (start 14.775 8.95) (end 13.5 10.225) (width 0.2) (layer "F.Cu") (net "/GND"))
 (via (at 10 14) (size 0.6) (drill 0.3) (layers "F.Cu" "B.Cu") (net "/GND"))
 (segment (start 11.875 5.45) (end 11.875 5.1748) (width 0.2) (layer "F.Cu") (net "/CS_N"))
 (segment (start 4.0024 11.3283) (end 6.175 13.5009) (width 0.2) (layer "F.Cu") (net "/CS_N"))
 (segment (start 11.875 5.1748) (end 10.3375 3.6373) (width 0.2) (layer "F.Cu") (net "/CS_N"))
 (segment (start 10.3375 3.6373) (end 5.9619 3.6373) (width 0.2) (layer "F.Cu") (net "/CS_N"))
 (segment (start 11.875 5.45) (end 11.875 6.7125) (width 0.2) (layer "F.Cu") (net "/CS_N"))
 (segment (start 4.0024 5.5968) (end 4.0024 11.3283) (width 0.2) (layer "F.Cu") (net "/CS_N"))
 (segment (start 11.875 6.7125) (end 10.5 8.0875) (width 0.2) (layer "F.Cu") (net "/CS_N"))
 (segment (start 5.9619 3.6373) (end 4.0024 5.5968) (width 0.2) (layer "F.Cu") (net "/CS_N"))
 (segment (start 6.175 13.5009) (end 6.175 14) (width 0.2) (layer "F.Cu") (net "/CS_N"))
 (segment (start 8.8375 8.25) (end 8.2827 7.6952) (width 0.2) (layer "F.Cu") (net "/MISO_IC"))
 (segment (start 4.675 8) (end 4.675 8.4711) (width 0.2) (layer "F.Cu") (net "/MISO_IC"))
 (segment (start 4.675 8.4711) (end 5.1361 8.9322) (width 0.2) (layer "F.Cu") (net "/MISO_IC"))
 (via (at 5.1361 8.9322) (size 0.6) (drill 0.3) (layers "F.Cu" "B.Cu") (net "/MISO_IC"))
 (via (at 8.2827 7.6952) (size 0.6) (drill 0.3) (layers "F.Cu" "B.Cu") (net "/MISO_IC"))
 (segment (start 5.1361 8.9322) (end 7.0457 8.9322) (width 0.2) (layer "B.Cu") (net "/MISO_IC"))
 (segment (start 7.0457 8.9322) (end 8.2827 7.6952) (width 0.2) (layer "B.Cu") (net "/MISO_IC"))
 (segment (start 13.125 5.1748) (end 11.0357 3.0855) (width 0.2) (layer "F.Cu") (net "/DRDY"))
 (segment (start 11.0357 3.0855) (end 9.1783 3.0855) (width 0.2) (layer "F.Cu") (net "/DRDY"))
 (segment (start 13.125 5.45) (end 13.125 5.1748) (width 0.2) (layer "F.Cu") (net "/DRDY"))
 (segment (start 8.1225 9.75) (end 8.8375 9.75) (width 0.2) (layer "F.Cu") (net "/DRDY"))
 (segment (start 8.04 9.6675) (end 8.1225 9.75) (width 0.2) (layer "F.Cu") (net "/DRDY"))
 (via (at 8.04 9.6675) (size 0.6) (drill 0.3) (layers "F.Cu" "B.Cu") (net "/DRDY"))
 (via (at 9.1783 3.0855) (size 0.6) (drill 0.3) (layers "F.Cu" "B.Cu") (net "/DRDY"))
 (segment (start 8.04 9.6675) (end 9.1783 8.5292) (width 0.2) (layer "B.Cu") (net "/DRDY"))
 (segment (start 9.1783 8.5292) (end 9.1783 3.0855) (width 0.2) (layer "B.Cu") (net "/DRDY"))
 (segment (start 8.125 5.45) (end 8.125 5.1726) (width 0.2) (layer "F.Cu") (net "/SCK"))
 (segment (start 8.125 5.1726) (end 8.9569 4.3407) (width 0.2) (layer "F.Cu") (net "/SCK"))
 (segment (start 8.9569 4.3407) (end 9.7266 4.3407) (width 0.2) (layer "F.Cu") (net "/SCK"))
 (segment (start 10 4.6141) (end 10 8.0875) (width 0.2) (layer "F.Cu") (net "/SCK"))
 (segment (start 9.7266 4.3407) (end 10 4.6141) (width 0.2) (layer "F.Cu") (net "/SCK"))
 (segment (start 9.5 8.0875) (end 9.5 5.575) (width 0.2) (layer "F.Cu") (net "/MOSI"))
 (segment (start 9.5 5.575) (end 9.375 5.45) (width 0.2) (layer "F.Cu") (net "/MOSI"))
 (segment (start 6.8719 3.989) (end 6.25 4.6109) (width 0.2) (layer "F.Cu") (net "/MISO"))
 (segment (start 9.8722 3.989) (end 6.8719 3.989) (width 0.2) (layer "F.Cu") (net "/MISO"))
 (segment (start 6.25 4.6109) (end 6.25 7.925) (width 0.2) (layer "F.Cu") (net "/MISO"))
 (segment (start 10.625 4.7418) (end 9.8722 3.989) (width 0.2) (layer "F.Cu") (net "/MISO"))
 (segment (start 10.625 5.45) (end 10.625 4.7418) (width 0.2) (layer "F.Cu") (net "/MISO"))
 (segment (start 6.25 7.925) (end 6.325 8) (width 0.2) (layer "F.Cu") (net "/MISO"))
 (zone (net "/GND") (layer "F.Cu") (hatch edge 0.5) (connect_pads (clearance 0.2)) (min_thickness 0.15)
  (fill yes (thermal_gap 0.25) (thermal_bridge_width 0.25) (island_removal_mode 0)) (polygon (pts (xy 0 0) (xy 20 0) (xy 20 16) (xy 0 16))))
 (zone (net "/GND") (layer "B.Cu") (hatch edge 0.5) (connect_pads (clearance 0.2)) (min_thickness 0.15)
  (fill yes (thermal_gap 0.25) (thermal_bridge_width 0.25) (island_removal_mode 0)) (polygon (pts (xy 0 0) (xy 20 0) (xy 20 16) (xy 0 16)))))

